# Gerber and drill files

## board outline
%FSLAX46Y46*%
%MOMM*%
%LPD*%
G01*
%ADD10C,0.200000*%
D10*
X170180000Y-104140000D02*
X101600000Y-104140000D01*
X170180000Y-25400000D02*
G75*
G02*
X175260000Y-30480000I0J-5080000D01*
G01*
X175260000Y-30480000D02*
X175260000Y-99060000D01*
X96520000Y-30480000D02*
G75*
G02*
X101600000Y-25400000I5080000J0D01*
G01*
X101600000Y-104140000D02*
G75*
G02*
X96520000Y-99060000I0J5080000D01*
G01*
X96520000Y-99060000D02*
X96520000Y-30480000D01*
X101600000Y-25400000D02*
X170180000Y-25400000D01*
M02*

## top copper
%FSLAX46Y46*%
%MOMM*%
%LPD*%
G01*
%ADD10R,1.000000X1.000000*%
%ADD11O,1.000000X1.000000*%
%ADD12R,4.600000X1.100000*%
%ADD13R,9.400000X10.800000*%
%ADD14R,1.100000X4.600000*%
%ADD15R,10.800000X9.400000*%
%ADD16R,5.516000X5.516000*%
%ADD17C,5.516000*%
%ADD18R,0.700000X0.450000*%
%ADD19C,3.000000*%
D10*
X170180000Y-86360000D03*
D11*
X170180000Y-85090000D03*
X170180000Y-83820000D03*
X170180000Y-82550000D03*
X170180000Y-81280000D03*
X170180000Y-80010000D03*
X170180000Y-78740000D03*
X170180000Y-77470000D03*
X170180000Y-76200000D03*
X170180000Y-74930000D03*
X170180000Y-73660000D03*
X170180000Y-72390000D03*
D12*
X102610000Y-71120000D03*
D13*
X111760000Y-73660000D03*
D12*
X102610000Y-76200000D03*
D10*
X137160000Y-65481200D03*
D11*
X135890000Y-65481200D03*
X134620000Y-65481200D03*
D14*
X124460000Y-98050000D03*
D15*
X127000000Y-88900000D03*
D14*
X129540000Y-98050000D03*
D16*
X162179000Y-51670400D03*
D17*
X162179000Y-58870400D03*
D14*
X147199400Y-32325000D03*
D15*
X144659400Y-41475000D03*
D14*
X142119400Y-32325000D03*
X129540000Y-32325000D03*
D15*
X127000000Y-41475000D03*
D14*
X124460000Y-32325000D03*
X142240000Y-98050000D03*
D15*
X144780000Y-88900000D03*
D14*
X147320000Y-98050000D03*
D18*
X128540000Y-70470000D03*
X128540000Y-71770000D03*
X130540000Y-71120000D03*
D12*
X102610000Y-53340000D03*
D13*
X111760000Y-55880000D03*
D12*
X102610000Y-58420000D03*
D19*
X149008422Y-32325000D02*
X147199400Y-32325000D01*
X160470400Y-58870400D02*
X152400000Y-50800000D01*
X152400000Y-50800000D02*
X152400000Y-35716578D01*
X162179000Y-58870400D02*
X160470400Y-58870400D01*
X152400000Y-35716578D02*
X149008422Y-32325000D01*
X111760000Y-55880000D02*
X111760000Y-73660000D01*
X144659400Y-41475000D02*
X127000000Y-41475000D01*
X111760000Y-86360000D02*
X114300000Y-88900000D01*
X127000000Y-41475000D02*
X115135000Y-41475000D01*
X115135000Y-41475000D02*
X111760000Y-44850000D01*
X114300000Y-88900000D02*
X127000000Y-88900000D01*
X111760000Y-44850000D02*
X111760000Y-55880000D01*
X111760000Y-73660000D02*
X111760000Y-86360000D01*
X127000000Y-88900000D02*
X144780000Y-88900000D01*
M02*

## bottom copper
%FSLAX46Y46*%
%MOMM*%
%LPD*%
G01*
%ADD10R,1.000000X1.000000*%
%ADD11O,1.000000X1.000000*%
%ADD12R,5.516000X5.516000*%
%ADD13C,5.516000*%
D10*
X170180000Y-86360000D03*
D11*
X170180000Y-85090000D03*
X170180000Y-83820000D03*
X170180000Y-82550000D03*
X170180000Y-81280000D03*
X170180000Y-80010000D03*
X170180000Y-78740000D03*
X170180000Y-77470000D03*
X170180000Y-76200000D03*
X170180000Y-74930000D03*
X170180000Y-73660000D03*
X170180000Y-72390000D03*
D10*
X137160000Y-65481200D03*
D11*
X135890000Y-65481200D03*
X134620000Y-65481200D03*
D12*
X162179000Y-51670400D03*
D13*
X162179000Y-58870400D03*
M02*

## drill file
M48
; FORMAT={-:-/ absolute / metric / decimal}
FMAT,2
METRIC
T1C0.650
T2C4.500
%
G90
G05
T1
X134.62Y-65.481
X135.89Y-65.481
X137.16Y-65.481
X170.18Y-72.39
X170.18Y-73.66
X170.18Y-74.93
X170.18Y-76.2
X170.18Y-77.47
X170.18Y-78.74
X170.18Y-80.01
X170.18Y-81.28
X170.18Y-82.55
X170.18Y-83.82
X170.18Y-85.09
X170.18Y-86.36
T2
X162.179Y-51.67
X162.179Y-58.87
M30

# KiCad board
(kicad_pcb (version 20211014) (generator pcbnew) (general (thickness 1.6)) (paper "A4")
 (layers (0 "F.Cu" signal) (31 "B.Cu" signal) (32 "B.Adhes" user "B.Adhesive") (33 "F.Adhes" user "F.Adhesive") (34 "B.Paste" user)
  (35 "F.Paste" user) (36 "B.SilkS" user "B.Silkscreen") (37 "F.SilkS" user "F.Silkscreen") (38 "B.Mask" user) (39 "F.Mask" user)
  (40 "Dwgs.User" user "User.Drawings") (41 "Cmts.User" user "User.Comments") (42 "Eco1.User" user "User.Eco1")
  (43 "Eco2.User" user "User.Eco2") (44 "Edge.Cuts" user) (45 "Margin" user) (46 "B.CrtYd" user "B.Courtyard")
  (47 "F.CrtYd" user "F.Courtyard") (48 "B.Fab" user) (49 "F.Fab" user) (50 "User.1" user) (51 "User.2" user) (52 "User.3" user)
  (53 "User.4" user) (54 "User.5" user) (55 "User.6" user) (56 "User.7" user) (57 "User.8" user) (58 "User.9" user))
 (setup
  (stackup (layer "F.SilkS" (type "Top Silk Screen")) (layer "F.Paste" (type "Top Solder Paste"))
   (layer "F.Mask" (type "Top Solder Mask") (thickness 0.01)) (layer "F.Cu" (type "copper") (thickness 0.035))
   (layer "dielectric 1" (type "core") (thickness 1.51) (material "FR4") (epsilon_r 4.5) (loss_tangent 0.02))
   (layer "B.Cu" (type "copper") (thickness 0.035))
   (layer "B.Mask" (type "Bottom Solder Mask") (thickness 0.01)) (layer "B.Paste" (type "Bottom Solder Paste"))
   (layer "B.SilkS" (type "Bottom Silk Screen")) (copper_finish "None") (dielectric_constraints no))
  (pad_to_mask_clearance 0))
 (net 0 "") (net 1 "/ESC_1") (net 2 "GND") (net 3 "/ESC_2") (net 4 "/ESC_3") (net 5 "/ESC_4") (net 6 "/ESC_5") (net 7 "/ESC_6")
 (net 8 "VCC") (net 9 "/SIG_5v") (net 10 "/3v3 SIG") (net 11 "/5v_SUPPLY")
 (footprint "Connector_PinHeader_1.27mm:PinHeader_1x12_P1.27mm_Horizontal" (layer "F.Cu") (at 170.18 86.36 180)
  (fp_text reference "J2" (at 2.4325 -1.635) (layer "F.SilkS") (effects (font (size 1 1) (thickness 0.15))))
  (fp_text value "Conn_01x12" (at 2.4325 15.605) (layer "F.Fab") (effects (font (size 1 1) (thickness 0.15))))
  (pad "1" thru_hole rect locked (at 0 0 180) (size 1 1) (drill 0.65) (layers *.Cu *.Mask) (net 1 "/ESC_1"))
  (pad "2" thru_hole oval locked (at 0 1.27 180) (size 1 1) (drill 0.65) (layers *.Cu *.Mask) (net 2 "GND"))
  (pad "3" thru_hole oval locked (at 0 2.54 180) (size 1 1) (drill 0.65) (layers *.Cu *.Mask) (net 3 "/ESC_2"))
  (pad "4" thru_hole oval locked (at 0 3.81 180) (size 1 1) (drill 0.65) (layers *.Cu *.Mask) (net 2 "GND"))
  (pad "5" thru_hole oval locked (at 0 5.08 180) (size 1 1) (drill 0.65) (layers *.Cu *.Mask) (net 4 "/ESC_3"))
  (pad "6" thru_hole oval locked (at 0 6.35 180) (size 1 1) (drill 0.65) (layers *.Cu *.Mask) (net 2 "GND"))
  (pad "7" thru_hole oval locked (at 0 7.62 180) (size 1 1) (drill 0.65) (layers *.Cu *.Mask) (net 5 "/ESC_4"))
  (pad "8" thru_hole oval locked (at 0 8.89 180) (size 1 1) (drill 0.65) (layers *.Cu *.Mask) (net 2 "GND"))
  (pad "9" thru_hole oval locked (at 0 10.16 180) (size 1 1) (drill 0.65) (layers *.Cu *.Mask) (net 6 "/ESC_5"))
  (pad "10" thru_hole oval locked (at 0 11.43 180) (size 1 1) (drill 0.65) (layers *.Cu *.Mask) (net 2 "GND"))
  (pad "11" thru_hole oval locked (at 0 12.7 180) (size 1 1) (drill 0.65) (layers *.Cu *.Mask) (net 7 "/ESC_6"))
  (pad "12" thru_hole oval locked (at 0 13.97 180) (size 1 1) (drill 0.65) (layers *.Cu *.Mask) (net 2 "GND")))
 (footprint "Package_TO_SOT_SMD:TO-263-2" (layer "F.Cu") (at 108.385 73.66)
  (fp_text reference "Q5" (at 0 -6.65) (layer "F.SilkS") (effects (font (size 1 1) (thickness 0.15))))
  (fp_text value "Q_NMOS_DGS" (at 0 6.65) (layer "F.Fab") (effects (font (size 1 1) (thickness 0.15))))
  (pad "" smd rect locked (at 5.8 2.775) (size 4.55 5.25) (layers "F.Paste"))
  (pad "" smd rect locked (at 0.95 -2.775) (size 4.55 5.25) (layers "F.Paste"))
  (pad "" smd rect locked (at 5.8 -2.775) (size 4.55 5.25) (layers "F.Paste"))
  (pad "" smd rect locked (at 0.95 2.775) (size 4.55 5.25) (layers "F.Paste"))
  (pad "1" smd rect locked (at -5.775 -2.54) (size 4.6 1.1) (layers "F.Cu" "F.Paste" "F.Mask") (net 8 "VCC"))
  (pad "2" smd rect locked (at 3.375 0) (size 9.4 10.8) (layers "F.Cu" "F.Mask") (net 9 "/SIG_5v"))
  (pad "3" smd rect locked (at -5.775 2.54) (size 4.6 1.1) (layers "F.Cu" "F.Paste" "F.Mask") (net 6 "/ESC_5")))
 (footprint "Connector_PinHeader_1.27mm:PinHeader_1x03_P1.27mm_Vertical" (layer "F.Cu") (at 137.16 65.4812 -90)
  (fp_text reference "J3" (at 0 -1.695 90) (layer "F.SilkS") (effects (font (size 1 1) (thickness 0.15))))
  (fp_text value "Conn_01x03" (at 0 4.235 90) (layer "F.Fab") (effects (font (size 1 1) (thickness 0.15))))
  (pad "1" thru_hole rect locked (at 0 0 270) (size 1 1) (drill 0.65) (layers *.Cu *.Mask) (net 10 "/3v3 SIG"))
  (pad "2" thru_hole oval locked (at 0 1.27 270) (size 1 1) (drill 0.65) (layers *.Cu *.Mask) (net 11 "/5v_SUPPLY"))
  (pad "3" thru_hole oval locked (at 0 2.54 270) (size 1 1) (drill 0.65) (layers *.Cu *.Mask) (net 2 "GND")))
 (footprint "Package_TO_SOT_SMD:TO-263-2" (layer "F.Cu") (at 127 92.275 90)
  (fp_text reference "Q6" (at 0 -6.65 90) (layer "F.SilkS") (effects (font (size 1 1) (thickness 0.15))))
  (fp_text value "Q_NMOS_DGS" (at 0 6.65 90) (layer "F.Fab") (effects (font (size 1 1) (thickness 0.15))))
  (pad "" smd rect locked (at 0.95 -2.775 90) (size 4.55 5.25) (layers "F.Paste"))
  (pad "" smd rect locked (at 0.95 2.775 90) (size 4.55 5.25) (layers "F.Paste"))
  (pad "" smd rect locked (at 5.8 2.775 90) (size 4.55 5.25) (layers "F.Paste"))
  (pad "" smd rect locked (at 5.8 -2.775 90) (size 4.55 5.25) (layers "F.Paste"))
  (pad "1" smd rect locked (at -5.775 -2.54 90) (size 4.6 1.1) (layers "F.Cu" "F.Paste" "F.Mask") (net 8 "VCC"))
  (pad "2" smd rect locked (at 3.375 0 90) (size 9.4 10.8) (layers "F.Cu" "F.Mask") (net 9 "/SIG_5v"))
  (pad "3" smd rect locked (at -5.775 2.54 90) (size 4.6 1.1) (layers "F.Cu" "F.Paste" "F.Mask") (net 4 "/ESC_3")))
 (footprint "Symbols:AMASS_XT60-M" (layer "F.Cu") (at 162.179 55.2704 -90)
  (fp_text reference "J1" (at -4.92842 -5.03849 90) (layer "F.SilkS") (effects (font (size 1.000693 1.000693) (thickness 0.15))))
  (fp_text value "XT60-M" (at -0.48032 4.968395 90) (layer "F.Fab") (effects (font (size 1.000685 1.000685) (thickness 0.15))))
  (pad "1" thru_hole rect locked (at -3.6 0 270) (size 5.516 5.516) (drill 4.5) (layers *.Cu *.Mask) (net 2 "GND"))
  (pad "2" thru_hole circle locked (at 3.6 0 270) (size 5.516 5.516) (drill 4.5) (layers *.Cu *.Mask) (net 8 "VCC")))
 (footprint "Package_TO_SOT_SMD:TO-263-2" (layer "F.Cu") (at 144.6594 38.1 -90)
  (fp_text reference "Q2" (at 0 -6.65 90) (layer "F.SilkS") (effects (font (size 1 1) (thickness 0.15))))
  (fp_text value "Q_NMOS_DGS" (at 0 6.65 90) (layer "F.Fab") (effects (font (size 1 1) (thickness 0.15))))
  (pad "" smd rect locked (at 0.95 2.775 270) (size 4.55 5.25) (layers "F.Paste"))
  (pad "" smd rect locked (at 0.95 -2.775 270) (size 4.55 5.25) (layers "F.Paste"))
  (pad "" smd rect locked (at 5.8 -2.775 270) (size 4.55 5.25) (layers "F.Paste"))
  (pad "" smd rect locked (at 5.8 2.775 270) (size 4.55 5.25) (layers "F.Paste"))
  (pad "1" smd rect locked (at -5.775 -2.54 270) (size 4.6 1.1) (layers "F.Cu" "F.Paste" "F.Mask") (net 8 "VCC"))
  (pad "2" smd rect locked (at 3.375 0 270) (size 9.4 10.8) (layers "F.Cu" "F.Mask") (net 9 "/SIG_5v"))
  (pad "3" smd rect locked (at -5.775 2.54 270) (size 4.6 1.1) (layers "F.Cu" "F.Paste" "F.Mask") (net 1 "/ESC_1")))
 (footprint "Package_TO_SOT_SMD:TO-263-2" (layer "F.Cu") (at 127 38.1 -90)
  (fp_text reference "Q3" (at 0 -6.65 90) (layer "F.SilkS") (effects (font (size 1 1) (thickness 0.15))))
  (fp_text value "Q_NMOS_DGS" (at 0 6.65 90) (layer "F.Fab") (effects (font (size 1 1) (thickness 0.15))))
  (pad "" smd rect locked (at 0.95 2.775 270) (size 4.55 5.25) (layers "F.Paste"))
  (pad "" smd rect locked (at 5.8 -2.775 270) (size 4.55 5.25) (layers "F.Paste"))
  (pad "" smd rect locked (at 5.8 2.775 270) (size 4.55 5.25) (layers "F.Paste"))
  (pad "" smd rect locked (at 0.95 -2.775 270) (size 4.55 5.25) (layers "F.Paste"))
  (pad "1" smd rect locked (at -5.775 -2.54 270) (size 4.6 1.1) (layers "F.Cu" "F.Paste" "F.Mask") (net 8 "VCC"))
  (pad "2" smd rect locked (at 3.375 0 270) (size 9.4 10.8) (layers "F.Cu" "F.Mask") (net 9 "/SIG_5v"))
  (pad "3" smd rect locked (at -5.775 2.54 270) (size 4.6 1.1) (layers "F.Cu" "F.Paste" "F.Mask") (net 5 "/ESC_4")))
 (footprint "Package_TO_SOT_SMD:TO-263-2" (layer "F.Cu") (at 144.78 92.275 90)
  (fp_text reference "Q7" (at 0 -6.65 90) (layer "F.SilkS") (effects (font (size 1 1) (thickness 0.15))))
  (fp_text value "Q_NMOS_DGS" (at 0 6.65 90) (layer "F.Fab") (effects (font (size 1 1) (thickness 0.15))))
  (pad "" smd rect locked (at 5.8 -2.775 90) (size 4.55 5.25) (layers "F.Paste"))
  (pad "" smd rect locked (at 5.8 2.775 90) (size 4.55 5.25) (layers "F.Paste"))
  (pad "" smd rect locked (at 0.95 -2.775 90) (size 4.55 5.25) (layers "F.Paste"))
  (pad "" smd rect locked (at 0.95 2.775 90) (size 4.55 5.25) (layers "F.Paste"))
  (pad "1" smd rect locked (at -5.775 -2.54 90) (size 4.6 1.1) (layers "F.Cu" "F.Paste" "F.Mask") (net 8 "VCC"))
  (pad "2" smd rect locked (at 3.375 0 90) (size 9.4 10.8) (layers "F.Cu" "F.Mask") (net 9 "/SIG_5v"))
  (pad "3" smd rect locked (at -5.775 2.54 90) (size 4.6 1.1) (layers "F.Cu" "F.Paste" "F.Mask") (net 7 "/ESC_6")))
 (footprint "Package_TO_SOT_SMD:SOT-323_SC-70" (layer "F.Cu") (at 129.54 71.12)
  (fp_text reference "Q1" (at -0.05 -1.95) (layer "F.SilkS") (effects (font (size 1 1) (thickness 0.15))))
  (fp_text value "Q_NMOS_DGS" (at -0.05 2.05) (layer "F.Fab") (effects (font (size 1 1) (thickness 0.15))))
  (pad "1" smd rect locked (at -1 -0.65 270) (size 0.45 0.7) (layers "F.Cu" "F.Paste" "F.Mask") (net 11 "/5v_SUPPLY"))
  (pad "2" smd rect locked (at -1 0.65 270) (size 0.45 0.7) (layers "F.Cu" "F.Paste" "F.Mask") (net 10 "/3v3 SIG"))
  (pad "3" smd rect locked (at 1 0 270) (size 0.45 0.7) (layers "F.Cu" "F.Paste" "F.Mask") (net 9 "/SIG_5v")))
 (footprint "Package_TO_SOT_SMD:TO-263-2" (layer "F.Cu") (at 108.385 55.88)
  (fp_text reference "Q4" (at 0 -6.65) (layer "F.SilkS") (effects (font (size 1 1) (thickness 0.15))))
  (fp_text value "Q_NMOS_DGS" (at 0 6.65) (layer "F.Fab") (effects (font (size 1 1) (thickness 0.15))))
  (pad "" smd rect locked (at 5.8 -2.775) (size 4.55 5.25) (layers "F.Paste"))
  (pad "" smd rect locked (at 0.95 2.775) (size 4.55 5.25) (layers "F.Paste"))
  (pad "" smd rect locked (at 5.8 2.775) (size 4.55 5.25) (layers "F.Paste"))
  (pad "" smd rect locked (at 0.95 -2.775) (size 4.55 5.25) (layers "F.Paste"))
  (pad "1" smd rect locked (at -5.775 -2.54) (size 4.6 1.1) (layers "F.Cu" "F.Paste" "F.Mask") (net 8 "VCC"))
  (pad "2" smd rect locked (at 3.375 0) (size 9.4 10.8) (layers "F.Cu" "F.Mask") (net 9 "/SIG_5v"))
  (pad "3" smd rect locked (at -5.775 2.54) (size 4.6 1.1) (layers "F.Cu" "F.Paste" "F.Mask") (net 3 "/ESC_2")))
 (gr_line (start 170.18 104.14) (end 101.6 104.14) (layer "Edge.Cuts") (width 0.2))
 (gr_arc (start 170.18 25.4) (mid 173.772102 26.887898) (end 175.26 30.48) (layer "Edge.Cuts") (width 0.2))
 (gr_line (start 175.26 30.48) (end 175.26 99.06) (layer "Edge.Cuts") (width 0.2))
 (gr_arc (start 96.52 30.48) (mid 98.007898 26.887898) (end 101.6 25.4) (layer "Edge.Cuts") (width 0.2))
 (gr_arc (start 101.6 104.14) (mid 98.007898 102.652102) (end 96.52 99.06) (layer "Edge.Cuts") (width 0.2))
 (gr_line (start 96.52 99.06) (end 96.52 30.48) (layer "Edge.Cuts") (width 0.2))
 (gr_line (start 101.6 25.4) (end 170.18 25.4) (layer "Edge.Cuts") (width 0.2))
 (segment (start 149.008422 32.325) (end 147.1994 32.325) (width 3) (layer "F.Cu") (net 8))
 (segment (start 160.4704 58.8704) (end 152.4 50.8) (width 3) (layer "F.Cu") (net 8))
 (segment (start 152.4 50.8) (end 152.4 35.716578) (width 3) (layer "F.Cu") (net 8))
 (segment (start 162.179 58.8704) (end 160.4704 58.8704) (width 3) (layer "F.Cu") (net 8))
 (segment (start 152.4 35.716578) (end 149.008422 32.325) (width 3) (layer "F.Cu") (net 8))
 (segment (start 111.76 55.88) (end 111.76 73.66) (width 3) (layer "F.Cu") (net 9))
 (segment (start 144.6594 41.475) (end 127 41.475) (width 3) (layer "F.Cu") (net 9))
 (segment (start 111.76 86.36) (end 114.3 88.9) (width 3) (layer "F.Cu") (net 9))
 (segment (start 127 41.475) (end 115.135 41.475) (width 3) (layer "F.Cu") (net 9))
 (segment (start 115.135 41.475) (end 111.76 44.85) (width 3) (layer "F.Cu") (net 9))
 (segment (start 114.3 88.9) (end 127 88.9) (width 3) (layer "F.Cu") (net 9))
 (segment (start 111.76 44.85) (end 111.76 55.88) (width 3) (layer "F.Cu") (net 9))
 (segment (start 111.76 73.66) (end 111.76 86.36) (width 3) (layer "F.Cu") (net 9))
 (segment (start 127 88.9) (end 144.78 88.9) (width 3) (layer "F.Cu") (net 9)))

